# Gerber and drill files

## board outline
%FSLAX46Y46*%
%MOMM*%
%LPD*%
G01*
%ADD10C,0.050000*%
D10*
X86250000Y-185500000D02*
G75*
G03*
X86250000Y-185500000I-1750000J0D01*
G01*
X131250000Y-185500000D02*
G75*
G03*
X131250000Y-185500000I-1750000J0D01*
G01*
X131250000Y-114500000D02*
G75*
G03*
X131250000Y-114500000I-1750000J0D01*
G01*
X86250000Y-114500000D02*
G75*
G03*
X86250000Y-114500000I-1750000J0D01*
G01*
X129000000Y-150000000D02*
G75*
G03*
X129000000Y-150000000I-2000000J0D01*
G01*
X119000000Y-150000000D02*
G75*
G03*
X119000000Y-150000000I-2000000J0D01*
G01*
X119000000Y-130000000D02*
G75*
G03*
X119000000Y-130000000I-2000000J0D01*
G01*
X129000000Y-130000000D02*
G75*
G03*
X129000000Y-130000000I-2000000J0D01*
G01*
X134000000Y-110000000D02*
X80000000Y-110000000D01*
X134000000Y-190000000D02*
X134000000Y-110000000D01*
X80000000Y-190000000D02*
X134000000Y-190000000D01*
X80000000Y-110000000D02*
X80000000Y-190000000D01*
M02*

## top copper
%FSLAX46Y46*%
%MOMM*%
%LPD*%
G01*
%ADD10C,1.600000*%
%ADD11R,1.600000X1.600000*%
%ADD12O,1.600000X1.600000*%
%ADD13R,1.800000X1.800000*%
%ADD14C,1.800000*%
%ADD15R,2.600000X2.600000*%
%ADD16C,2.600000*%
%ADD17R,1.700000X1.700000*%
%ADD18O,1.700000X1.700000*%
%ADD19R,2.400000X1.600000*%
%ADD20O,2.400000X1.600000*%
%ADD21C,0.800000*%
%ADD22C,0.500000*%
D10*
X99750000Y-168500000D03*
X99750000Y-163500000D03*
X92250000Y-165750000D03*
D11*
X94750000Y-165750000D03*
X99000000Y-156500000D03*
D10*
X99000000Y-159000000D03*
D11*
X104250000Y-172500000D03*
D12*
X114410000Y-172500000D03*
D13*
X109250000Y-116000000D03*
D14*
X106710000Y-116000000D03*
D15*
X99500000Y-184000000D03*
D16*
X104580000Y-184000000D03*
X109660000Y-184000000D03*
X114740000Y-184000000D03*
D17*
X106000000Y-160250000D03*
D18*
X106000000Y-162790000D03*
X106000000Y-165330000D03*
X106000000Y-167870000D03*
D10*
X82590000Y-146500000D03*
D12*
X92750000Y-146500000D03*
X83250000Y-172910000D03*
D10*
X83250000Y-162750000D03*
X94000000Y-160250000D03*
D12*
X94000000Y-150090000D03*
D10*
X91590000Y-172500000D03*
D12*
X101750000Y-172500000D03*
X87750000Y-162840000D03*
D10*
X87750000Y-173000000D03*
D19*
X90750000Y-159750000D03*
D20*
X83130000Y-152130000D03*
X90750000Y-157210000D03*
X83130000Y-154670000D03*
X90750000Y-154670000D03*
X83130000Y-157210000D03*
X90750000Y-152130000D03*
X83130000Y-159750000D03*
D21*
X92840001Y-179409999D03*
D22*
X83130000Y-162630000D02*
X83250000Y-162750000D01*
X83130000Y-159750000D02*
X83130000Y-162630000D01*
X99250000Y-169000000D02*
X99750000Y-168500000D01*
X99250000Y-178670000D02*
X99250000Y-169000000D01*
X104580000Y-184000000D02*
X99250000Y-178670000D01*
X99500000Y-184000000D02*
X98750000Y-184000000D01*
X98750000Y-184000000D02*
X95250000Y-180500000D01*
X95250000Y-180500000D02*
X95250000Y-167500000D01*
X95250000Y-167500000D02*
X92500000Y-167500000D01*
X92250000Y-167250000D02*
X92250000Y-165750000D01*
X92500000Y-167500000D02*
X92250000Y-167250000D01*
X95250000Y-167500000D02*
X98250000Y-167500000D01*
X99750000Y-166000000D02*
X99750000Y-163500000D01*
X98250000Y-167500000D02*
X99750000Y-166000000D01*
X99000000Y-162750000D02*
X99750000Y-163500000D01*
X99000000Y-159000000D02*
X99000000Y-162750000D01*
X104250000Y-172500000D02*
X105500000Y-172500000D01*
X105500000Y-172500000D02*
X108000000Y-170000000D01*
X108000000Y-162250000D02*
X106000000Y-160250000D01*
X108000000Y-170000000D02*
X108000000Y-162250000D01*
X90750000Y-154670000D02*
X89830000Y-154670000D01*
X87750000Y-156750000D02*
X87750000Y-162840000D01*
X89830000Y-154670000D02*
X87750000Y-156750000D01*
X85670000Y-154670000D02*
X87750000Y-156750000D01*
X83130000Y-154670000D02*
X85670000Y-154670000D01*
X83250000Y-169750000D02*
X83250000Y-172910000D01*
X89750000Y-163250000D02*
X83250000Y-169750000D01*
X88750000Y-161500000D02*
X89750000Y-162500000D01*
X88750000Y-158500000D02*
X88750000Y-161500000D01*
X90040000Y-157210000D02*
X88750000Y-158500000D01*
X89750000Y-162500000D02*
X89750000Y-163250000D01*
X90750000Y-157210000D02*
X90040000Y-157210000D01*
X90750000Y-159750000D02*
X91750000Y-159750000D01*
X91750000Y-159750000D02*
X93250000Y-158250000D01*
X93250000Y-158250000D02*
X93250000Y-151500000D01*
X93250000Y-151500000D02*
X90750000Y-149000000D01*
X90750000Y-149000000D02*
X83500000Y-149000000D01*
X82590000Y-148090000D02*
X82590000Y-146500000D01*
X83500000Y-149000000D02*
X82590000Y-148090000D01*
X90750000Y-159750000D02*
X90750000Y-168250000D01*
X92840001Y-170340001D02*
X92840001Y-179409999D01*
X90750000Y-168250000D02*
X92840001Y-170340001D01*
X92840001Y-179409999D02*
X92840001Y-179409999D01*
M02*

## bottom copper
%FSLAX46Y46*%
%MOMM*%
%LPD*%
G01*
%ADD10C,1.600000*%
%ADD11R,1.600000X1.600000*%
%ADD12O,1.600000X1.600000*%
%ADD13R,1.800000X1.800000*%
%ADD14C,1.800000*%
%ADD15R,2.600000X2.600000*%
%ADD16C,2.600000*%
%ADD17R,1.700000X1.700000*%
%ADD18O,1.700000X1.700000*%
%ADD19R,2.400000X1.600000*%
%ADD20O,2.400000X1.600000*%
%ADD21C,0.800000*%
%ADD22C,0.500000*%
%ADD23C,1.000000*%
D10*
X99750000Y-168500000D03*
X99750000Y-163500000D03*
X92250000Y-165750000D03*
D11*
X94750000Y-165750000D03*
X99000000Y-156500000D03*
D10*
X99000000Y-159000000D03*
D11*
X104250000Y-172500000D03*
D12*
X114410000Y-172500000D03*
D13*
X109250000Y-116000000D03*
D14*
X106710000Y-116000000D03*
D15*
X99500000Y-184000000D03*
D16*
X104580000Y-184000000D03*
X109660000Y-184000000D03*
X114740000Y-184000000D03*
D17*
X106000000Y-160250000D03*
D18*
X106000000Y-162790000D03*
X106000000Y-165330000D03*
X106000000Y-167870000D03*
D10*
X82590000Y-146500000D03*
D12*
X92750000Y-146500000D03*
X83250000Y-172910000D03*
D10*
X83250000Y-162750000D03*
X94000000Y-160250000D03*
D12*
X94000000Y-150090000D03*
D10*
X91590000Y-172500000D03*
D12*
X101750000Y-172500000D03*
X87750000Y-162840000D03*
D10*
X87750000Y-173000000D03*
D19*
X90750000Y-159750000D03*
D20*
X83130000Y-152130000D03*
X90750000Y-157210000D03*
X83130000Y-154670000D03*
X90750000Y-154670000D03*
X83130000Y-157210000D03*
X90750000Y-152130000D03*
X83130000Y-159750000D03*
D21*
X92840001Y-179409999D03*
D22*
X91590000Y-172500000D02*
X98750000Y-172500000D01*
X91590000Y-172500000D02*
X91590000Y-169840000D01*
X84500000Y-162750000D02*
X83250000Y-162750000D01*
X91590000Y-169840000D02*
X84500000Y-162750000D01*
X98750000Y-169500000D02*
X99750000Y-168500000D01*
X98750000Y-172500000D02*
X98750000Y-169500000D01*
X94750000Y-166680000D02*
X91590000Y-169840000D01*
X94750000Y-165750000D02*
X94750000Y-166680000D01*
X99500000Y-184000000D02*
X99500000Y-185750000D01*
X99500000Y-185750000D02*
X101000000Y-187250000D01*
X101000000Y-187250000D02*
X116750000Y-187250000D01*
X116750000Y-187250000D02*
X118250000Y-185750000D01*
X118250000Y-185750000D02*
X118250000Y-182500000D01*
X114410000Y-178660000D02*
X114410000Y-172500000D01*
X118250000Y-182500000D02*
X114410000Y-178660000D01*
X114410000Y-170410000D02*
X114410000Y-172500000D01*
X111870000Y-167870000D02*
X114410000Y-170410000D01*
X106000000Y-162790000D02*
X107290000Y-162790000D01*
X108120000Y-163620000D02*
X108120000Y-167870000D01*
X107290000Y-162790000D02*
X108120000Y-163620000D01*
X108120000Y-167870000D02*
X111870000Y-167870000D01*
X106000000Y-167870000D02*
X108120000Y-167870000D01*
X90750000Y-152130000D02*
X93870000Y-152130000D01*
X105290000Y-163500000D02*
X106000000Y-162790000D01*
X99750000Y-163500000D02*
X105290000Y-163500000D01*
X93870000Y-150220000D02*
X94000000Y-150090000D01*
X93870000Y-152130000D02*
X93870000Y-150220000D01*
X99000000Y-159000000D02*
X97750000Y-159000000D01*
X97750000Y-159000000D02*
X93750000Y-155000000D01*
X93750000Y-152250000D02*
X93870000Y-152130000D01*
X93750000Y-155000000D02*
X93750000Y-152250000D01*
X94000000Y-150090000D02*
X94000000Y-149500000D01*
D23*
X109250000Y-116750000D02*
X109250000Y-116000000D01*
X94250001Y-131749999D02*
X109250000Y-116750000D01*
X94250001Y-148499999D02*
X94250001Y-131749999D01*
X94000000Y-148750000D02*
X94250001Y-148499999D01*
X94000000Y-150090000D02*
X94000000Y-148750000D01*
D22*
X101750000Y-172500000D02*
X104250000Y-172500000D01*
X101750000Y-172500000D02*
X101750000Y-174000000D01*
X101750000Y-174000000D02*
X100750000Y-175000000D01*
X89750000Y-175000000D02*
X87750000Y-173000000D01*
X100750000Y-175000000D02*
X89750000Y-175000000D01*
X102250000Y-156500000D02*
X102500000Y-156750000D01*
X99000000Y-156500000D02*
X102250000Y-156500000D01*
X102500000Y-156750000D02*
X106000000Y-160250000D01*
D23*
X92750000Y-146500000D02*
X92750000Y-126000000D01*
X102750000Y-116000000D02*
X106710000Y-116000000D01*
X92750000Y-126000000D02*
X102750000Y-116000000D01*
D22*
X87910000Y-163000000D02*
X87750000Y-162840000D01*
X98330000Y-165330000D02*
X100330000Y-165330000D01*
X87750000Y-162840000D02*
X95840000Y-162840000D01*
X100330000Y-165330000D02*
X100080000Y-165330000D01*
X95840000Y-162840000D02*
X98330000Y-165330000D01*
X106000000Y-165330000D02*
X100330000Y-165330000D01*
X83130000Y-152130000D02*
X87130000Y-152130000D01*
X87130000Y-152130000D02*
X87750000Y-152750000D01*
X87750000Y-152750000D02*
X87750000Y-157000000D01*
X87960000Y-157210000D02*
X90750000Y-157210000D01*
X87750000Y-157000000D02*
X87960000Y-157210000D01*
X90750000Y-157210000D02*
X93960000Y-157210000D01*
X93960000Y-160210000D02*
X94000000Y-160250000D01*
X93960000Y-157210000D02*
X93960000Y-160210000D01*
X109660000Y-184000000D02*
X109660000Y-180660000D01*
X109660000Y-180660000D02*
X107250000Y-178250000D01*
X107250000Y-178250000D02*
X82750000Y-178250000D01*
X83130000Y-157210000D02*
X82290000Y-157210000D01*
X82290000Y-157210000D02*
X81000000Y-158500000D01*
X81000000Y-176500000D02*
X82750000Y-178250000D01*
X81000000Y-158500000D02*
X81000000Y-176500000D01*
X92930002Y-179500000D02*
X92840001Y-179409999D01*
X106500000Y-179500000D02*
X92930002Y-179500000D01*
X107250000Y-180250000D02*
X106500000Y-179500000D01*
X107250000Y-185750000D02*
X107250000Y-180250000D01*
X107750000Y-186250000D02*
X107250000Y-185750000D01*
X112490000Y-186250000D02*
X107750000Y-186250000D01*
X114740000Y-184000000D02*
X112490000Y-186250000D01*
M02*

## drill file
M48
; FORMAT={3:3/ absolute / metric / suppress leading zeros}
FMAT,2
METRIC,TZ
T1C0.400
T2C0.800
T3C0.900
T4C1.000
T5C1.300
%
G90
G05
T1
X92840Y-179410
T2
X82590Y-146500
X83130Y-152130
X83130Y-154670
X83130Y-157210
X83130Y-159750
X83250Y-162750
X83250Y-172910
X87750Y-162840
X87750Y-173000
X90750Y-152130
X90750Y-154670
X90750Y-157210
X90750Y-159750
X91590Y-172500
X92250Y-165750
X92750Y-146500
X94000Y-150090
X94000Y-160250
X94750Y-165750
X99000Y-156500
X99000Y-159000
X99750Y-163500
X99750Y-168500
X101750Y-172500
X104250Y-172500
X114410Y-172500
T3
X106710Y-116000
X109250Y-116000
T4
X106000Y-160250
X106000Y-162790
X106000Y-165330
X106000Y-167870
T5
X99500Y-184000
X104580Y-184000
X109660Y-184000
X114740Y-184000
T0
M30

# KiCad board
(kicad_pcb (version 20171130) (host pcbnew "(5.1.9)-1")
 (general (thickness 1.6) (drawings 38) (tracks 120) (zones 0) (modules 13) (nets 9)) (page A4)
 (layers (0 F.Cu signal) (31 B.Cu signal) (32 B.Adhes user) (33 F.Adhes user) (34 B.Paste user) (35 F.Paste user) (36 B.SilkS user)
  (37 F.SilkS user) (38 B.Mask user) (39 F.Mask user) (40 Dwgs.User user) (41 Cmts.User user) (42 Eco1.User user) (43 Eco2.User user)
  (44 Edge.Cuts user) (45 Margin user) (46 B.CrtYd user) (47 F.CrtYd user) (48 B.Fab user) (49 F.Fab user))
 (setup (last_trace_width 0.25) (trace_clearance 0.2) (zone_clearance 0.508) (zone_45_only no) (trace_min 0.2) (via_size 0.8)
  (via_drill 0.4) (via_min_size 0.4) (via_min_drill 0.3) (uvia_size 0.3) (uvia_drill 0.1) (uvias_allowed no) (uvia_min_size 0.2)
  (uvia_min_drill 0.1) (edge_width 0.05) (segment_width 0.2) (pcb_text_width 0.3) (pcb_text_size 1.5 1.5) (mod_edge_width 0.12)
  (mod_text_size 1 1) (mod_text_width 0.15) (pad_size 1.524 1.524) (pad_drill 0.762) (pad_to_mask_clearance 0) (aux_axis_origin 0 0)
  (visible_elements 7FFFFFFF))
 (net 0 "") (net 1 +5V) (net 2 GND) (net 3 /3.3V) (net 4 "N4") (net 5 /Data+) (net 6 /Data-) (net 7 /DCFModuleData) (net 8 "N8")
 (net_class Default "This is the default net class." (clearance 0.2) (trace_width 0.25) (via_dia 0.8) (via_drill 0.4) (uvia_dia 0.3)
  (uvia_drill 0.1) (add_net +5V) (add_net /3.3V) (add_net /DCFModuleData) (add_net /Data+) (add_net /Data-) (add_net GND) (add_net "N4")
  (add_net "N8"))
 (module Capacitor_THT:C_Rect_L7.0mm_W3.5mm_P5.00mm (layer F.Cu) (at 99.75 168.5 90)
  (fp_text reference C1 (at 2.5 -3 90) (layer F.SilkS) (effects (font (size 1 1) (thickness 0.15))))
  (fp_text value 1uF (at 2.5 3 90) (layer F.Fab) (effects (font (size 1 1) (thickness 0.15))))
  (pad 1 thru_hole circle (at 0 0 90) (size 1.6 1.6) (drill 0.8) (layers *.Cu *.Mask) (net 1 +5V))
  (pad 2 thru_hole circle (at 5 0 90) (size 1.6 1.6) (drill 0.8) (layers *.Cu *.Mask) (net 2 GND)))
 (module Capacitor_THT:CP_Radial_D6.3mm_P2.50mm (layer F.Cu) (at 94.75 165.75 180)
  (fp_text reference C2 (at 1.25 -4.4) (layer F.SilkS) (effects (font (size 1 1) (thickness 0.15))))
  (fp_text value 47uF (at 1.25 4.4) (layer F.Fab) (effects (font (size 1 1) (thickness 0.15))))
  (pad 2 thru_hole circle (at 2.5 0 180) (size 1.6 1.6) (drill 0.8) (layers *.Cu *.Mask) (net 2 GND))
  (pad 1 thru_hole rect (at 0 0 180) (size 1.6 1.6) (drill 0.8) (layers *.Cu *.Mask) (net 1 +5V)))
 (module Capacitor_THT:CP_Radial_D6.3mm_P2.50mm (layer F.Cu) (at 99 156.5 270)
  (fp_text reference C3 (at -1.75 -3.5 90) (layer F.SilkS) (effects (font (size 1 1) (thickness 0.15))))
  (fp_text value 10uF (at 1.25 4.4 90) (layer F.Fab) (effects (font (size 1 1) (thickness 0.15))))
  (pad 1 thru_hole rect (at 0 0 270) (size 1.6 1.6) (drill 0.8) (layers *.Cu *.Mask) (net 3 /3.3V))
  (pad 2 thru_hole circle (at 2.5 0 270) (size 1.6 1.6) (drill 0.8) (layers *.Cu *.Mask) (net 2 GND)))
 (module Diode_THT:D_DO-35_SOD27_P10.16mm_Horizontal (layer F.Cu) (at 104.25 172.5)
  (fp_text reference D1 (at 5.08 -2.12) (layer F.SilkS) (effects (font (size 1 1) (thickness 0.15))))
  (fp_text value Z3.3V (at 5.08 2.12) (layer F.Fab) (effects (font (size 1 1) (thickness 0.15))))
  (pad 1 thru_hole rect (at 0 0) (size 1.6 1.6) (drill 0.8) (layers *.Cu *.Mask) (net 3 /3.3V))
  (pad 2 thru_hole oval (at 10.16 0) (size 1.6 1.6) (drill 0.8) (layers *.Cu *.Mask) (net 2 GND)))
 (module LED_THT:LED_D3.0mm (layer F.Cu) (at 109.25 116 180)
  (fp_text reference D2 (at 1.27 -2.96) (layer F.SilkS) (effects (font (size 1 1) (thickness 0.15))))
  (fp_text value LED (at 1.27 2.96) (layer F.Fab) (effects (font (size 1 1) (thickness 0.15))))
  (pad 1 thru_hole rect (at 0 0 180) (size 1.8 1.8) (drill 0.9) (layers *.Cu *.Mask) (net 2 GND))
  (pad 2 thru_hole circle (at 2.54 0 180) (size 1.8 1.8) (drill 0.9) (layers *.Cu *.Mask) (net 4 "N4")))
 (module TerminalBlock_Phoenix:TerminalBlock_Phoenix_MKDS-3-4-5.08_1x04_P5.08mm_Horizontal (layer F.Cu) (at 99.5 184)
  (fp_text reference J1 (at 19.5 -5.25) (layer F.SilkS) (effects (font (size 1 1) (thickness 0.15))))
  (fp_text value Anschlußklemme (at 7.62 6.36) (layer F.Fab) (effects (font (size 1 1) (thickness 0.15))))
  (pad 1 thru_hole rect (at 0 0) (size 2.6 2.6) (drill 1.3) (layers *.Cu *.Mask) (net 2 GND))
  (pad 2 thru_hole circle (at 5.08 0) (size 2.6 2.6) (drill 1.3) (layers *.Cu *.Mask) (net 1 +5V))
  (pad 3 thru_hole circle (at 10.16 0) (size 2.6 2.6) (drill 1.3) (layers *.Cu *.Mask) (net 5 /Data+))
  (pad 4 thru_hole circle (at 15.24 0) (size 2.6 2.6) (drill 1.3) (layers *.Cu *.Mask) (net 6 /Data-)))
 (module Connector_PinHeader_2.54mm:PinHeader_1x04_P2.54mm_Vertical (layer F.Cu) (at 106 160.25)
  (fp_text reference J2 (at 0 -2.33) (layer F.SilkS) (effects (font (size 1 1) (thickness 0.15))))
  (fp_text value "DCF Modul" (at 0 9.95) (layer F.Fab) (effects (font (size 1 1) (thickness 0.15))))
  (pad 1 thru_hole rect (at 0 0) (size 1.7 1.7) (drill 1) (layers *.Cu *.Mask) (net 3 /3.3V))
  (pad 2 thru_hole oval (at 0 2.54) (size 1.7 1.7) (drill 1) (layers *.Cu *.Mask) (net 2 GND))
  (pad 3 thru_hole oval (at 0 5.08) (size 1.7 1.7) (drill 1) (layers *.Cu *.Mask) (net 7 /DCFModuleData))
  (pad 4 thru_hole oval (at 0 7.62) (size 1.7 1.7) (drill 1) (layers *.Cu *.Mask) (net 2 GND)))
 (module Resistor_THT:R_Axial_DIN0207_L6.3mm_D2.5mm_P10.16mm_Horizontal (layer F.Cu) (at 82.59 146.5)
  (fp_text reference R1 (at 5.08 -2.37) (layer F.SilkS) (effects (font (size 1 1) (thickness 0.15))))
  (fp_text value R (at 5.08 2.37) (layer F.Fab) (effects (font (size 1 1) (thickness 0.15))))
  (pad 1 thru_hole circle (at 0 0) (size 1.6 1.6) (drill 0.8) (layers *.Cu *.Mask) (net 6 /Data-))
  (pad 2 thru_hole oval (at 10.16 0) (size 1.6 1.6) (drill 0.8) (layers *.Cu *.Mask) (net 4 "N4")))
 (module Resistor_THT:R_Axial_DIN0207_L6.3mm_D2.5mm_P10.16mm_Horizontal (layer F.Cu) (at 83.25 162.75 270)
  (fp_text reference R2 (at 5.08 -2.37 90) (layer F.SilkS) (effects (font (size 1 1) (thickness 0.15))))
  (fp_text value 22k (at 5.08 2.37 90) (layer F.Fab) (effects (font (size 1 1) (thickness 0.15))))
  (pad 2 thru_hole oval (at 10.16 0 270) (size 1.6 1.6) (drill 0.8) (layers *.Cu *.Mask) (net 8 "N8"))
  (pad 1 thru_hole circle (at 0 0 270) (size 1.6 1.6) (drill 0.8) (layers *.Cu *.Mask) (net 1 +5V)))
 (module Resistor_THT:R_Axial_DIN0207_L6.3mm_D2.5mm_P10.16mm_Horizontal (layer F.Cu) (at 94 160.25 90)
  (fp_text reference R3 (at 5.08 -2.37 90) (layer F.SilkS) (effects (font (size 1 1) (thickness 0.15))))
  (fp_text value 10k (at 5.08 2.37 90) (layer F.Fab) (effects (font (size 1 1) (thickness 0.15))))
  (pad 1 thru_hole circle (at 0 0 90) (size 1.6 1.6) (drill 0.8) (layers *.Cu *.Mask) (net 8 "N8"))
  (pad 2 thru_hole oval (at 10.16 0 90) (size 1.6 1.6) (drill 0.8) (layers *.Cu *.Mask) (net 2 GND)))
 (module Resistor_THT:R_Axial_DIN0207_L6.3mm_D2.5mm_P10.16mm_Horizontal (layer F.Cu) (at 91.59 172.5)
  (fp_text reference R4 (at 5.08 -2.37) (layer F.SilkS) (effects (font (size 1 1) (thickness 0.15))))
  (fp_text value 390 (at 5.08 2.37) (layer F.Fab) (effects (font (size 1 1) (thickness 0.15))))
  (pad 1 thru_hole circle (at 0 0) (size 1.6 1.6) (drill 0.8) (layers *.Cu *.Mask) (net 1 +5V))
  (pad 2 thru_hole oval (at 10.16 0) (size 1.6 1.6) (drill 0.8) (layers *.Cu *.Mask) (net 3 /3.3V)))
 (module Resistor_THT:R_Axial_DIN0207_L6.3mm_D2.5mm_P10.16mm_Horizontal (layer F.Cu) (at 87.75 173 90)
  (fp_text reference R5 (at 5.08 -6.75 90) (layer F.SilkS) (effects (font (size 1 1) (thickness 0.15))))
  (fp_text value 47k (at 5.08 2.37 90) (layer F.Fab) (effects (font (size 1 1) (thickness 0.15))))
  (pad 2 thru_hole oval (at 10.16 0 90) (size 1.6 1.6) (drill 0.8) (layers *.Cu *.Mask) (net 7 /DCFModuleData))
  (pad 1 thru_hole circle (at 0 0 90) (size 1.6 1.6) (drill 0.8) (layers *.Cu *.Mask) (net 3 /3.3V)))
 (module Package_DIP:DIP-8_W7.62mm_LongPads (layer F.Cu) (at 90.75 159.75 180)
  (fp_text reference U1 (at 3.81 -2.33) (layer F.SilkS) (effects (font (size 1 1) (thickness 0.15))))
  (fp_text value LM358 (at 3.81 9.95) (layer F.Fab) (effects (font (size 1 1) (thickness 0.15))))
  (pad 1 thru_hole rect (at 0 0 180) (size 2.4 1.6) (drill 0.8) (layers *.Cu *.Mask) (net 6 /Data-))
  (pad 5 thru_hole oval (at 7.62 7.62 180) (size 2.4 1.6) (drill 0.8) (layers *.Cu *.Mask) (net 8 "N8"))
  (pad 2 thru_hole oval (at 0 2.54 180) (size 2.4 1.6) (drill 0.8) (layers *.Cu *.Mask) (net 8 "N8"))
  (pad 6 thru_hole oval (at 7.62 5.08 180) (size 2.4 1.6) (drill 0.8) (layers *.Cu *.Mask) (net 7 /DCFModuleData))
  (pad 3 thru_hole oval (at 0 5.08 180) (size 2.4 1.6) (drill 0.8) (layers *.Cu *.Mask) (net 7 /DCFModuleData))
  (pad 7 thru_hole oval (at 7.62 2.54 180) (size 2.4 1.6) (drill 0.8) (layers *.Cu *.Mask) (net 5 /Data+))
  (pad 4 thru_hole oval (at 0 7.62 180) (size 2.4 1.6) (drill 0.8) (layers *.Cu *.Mask) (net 2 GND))
  (pad 8 thru_hole oval (at 7.62 0 180) (size 2.4 1.6) (drill 0.8) (layers *.Cu *.Mask) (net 1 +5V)))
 (gr_circle (center 84.5 185.5) (end 86.25 185.5) (layer Edge.Cuts) (width 0.05))
 (gr_circle (center 129.5 185.5) (end 131.25 185.5) (layer Edge.Cuts) (width 0.05))
 (gr_circle (center 129.5 114.5) (end 131.25 114.5) (layer Edge.Cuts) (width 0.05))
 (gr_circle (center 84.5 114.5) (end 86.25 114.5) (layer Edge.Cuts) (width 0.05))
 (gr_circle (center 127 150) (end 129 150) (layer Edge.Cuts) (width 0.05))
 (gr_circle (center 117 150) (end 119 150) (layer Edge.Cuts) (width 0.05))
 (gr_circle (center 117 130) (end 119 130) (layer Edge.Cuts) (width 0.05))
 (gr_circle (center 127 130) (end 129 130) (layer Edge.Cuts) (width 0.05))
 (gr_line (start 134 110) (end 80 110) (layer Edge.Cuts) (width 0.05))
 (gr_line (start 134 190) (end 134 110) (layer Edge.Cuts) (width 0.05))
 (gr_line (start 80 190) (end 134 190) (layer Edge.Cuts) (width 0.05))
 (gr_line (start 80 110) (end 80 190) (layer Edge.Cuts) (width 0.05))
 (segment (start 91.59 172.5) (end 98.75 172.5) (width 0.5) (layer B.Cu) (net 1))
 (segment (start 83.13 162.63) (end 83.25 162.75) (width 0.5) (layer F.Cu) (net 1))
 (segment (start 83.13 159.75) (end 83.13 162.63) (width 0.5) (layer F.Cu) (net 1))
 (segment (start 91.59 172.5) (end 91.59 169.84) (width 0.5) (layer B.Cu) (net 1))
 (segment (start 84.5 162.75) (end 83.25 162.75) (width 0.5) (layer B.Cu) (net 1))
 (segment (start 91.59 169.84) (end 84.5 162.75) (width 0.5) (layer B.Cu) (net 1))
 (segment (start 98.75 169.5) (end 99.75 168.5) (width 0.5) (layer B.Cu) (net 1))
 (segment (start 98.75 172.5) (end 98.75 169.5) (width 0.5) (layer B.Cu) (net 1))
 (segment (start 99.25 169) (end 99.75 168.5) (width 0.5) (layer F.Cu) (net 1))
 (segment (start 99.25 178.67) (end 99.25 169) (width 0.5) (layer F.Cu) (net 1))
 (segment (start 104.58 184) (end 99.25 178.67) (width 0.5) (layer F.Cu) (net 1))
 (segment (start 94.75 166.68) (end 91.59 169.84) (width 0.5) (layer B.Cu) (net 1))
 (segment (start 94.75 165.75) (end 94.75 166.68) (width 0.5) (layer B.Cu) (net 1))
 (segment (start 99.5 184) (end 99.5 185.75) (width 0.5) (layer B.Cu) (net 2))
 (segment (start 99.5 185.75) (end 101 187.25) (width 0.5) (layer B.Cu) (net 2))
 (segment (start 101 187.25) (end 116.75 187.25) (width 0.5) (layer B.Cu) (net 2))
 (segment (start 116.75 187.25) (end 118.25 185.75) (width 0.5) (layer B.Cu) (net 2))
 (segment (start 118.25 185.75) (end 118.25 182.5) (width 0.5) (layer B.Cu) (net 2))
 (segment (start 114.41 178.66) (end 114.41 172.5) (width 0.5) (layer B.Cu) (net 2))
 (segment (start 118.25 182.5) (end 114.41 178.66) (width 0.5) (layer B.Cu) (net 2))
 (segment (start 114.41 170.41) (end 114.41 172.5) (width 0.5) (layer B.Cu) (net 2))
 (segment (start 111.87 167.87) (end 114.41 170.41) (width 0.5) (layer B.Cu) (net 2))
 (segment (start 106 162.79) (end 107.29 162.79) (width 0.5) (layer B.Cu) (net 2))
 (segment (start 108.12 163.62) (end 108.12 167.87) (width 0.5) (layer B.Cu) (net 2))
 (segment (start 107.29 162.79) (end 108.12 163.62) (width 0.5) (layer B.Cu) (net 2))
 (segment (start 108.12 167.87) (end 111.87 167.87) (width 0.5) (layer B.Cu) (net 2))
 (segment (start 106 167.87) (end 108.12 167.87) (width 0.5) (layer B.Cu) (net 2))
 (segment (start 99.5 184) (end 98.75 184) (width 0.5) (layer F.Cu) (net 2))
 (segment (start 98.75 184) (end 95.25 180.5) (width 0.5) (layer F.Cu) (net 2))
 (segment (start 95.25 180.5) (end 95.25 167.5) (width 0.5) (layer F.Cu) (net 2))
 (segment (start 90.75 152.13) (end 93.87 152.13) (width 0.5) (layer B.Cu) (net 2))
 (segment (start 105.29 163.5) (end 106 162.79) (width 0.5) (layer B.Cu) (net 2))
 (segment (start 99.75 163.5) (end 105.29 163.5) (width 0.5) (layer B.Cu) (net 2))
 (segment (start 95.25 167.5) (end 92.5 167.5) (width 0.5) (layer F.Cu) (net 2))
 (segment (start 92.25 167.25) (end 92.25 165.75) (width 0.5) (layer F.Cu) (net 2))
 (segment (start 92.5 167.5) (end 92.25 167.25) (width 0.5) (layer F.Cu) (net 2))
 (segment (start 95.25 167.5) (end 98.25 167.5) (width 0.5) (layer F.Cu) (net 2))
 (segment (start 99.75 166) (end 99.75 163.5) (width 0.5) (layer F.Cu) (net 2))
 (segment (start 98.25 167.5) (end 99.75 166) (width 0.5) (layer F.Cu) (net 2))
 (segment (start 93.87 150.22) (end 94 150.09) (width 0.5) (layer B.Cu) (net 2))
 (segment (start 93.87 152.13) (end 93.87 150.22) (width 0.5) (layer B.Cu) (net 2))
 (segment (start 99 159) (end 97.75 159) (width 0.5) (layer B.Cu) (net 2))
 (segment (start 97.75 159) (end 93.75 155) (width 0.5) (layer B.Cu) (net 2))
 (segment (start 93.75 152.25) (end 93.87 152.13) (width 0.5) (layer B.Cu) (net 2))
 (segment (start 93.75 155) (end 93.75 152.25) (width 0.5) (layer B.Cu) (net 2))
 (segment (start 99 162.75) (end 99.75 163.5) (width 0.5) (layer F.Cu) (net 2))
 (segment (start 99 159) (end 99 162.75) (width 0.5) (layer F.Cu) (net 2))
 (segment (start 94 150.09) (end 94 149.5) (width 0.5) (layer B.Cu) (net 2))
 (segment (start 109.25 116.75) (end 109.25 116) (width 1) (layer B.Cu) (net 2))
 (segment (start 94.250001 131.749999) (end 109.25 116.75) (width 1) (layer B.Cu) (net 2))
 (segment (start 94.250001 148.499999) (end 94.250001 131.749999) (width 1) (layer B.Cu) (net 2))
 (segment (start 94 148.75) (end 94.250001 148.499999) (width 1) (layer B.Cu) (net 2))
 (segment (start 94 150.09) (end 94 148.75) (width 1) (layer B.Cu) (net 2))
 (segment (start 104.25 172.5) (end 105.5 172.5) (width 0.5) (layer F.Cu) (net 3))
 (segment (start 105.5 172.5) (end 108 170) (width 0.5) (layer F.Cu) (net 3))
 (segment (start 108 162.25) (end 106 160.25) (width 0.5) (layer F.Cu) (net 3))
 (segment (start 108 170) (end 108 162.25) (width 0.5) (layer F.Cu) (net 3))
 (segment (start 101.75 172.5) (end 104.25 172.5) (width 0.5) (layer B.Cu) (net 3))
 (segment (start 101.75 172.5) (end 101.75 174) (width 0.5) (layer B.Cu) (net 3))
 (segment (start 101.75 174) (end 100.75 175) (width 0.5) (layer B.Cu) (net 3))
 (segment (start 89.75 175) (end 87.75 173) (width 0.5) (layer B.Cu) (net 3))
 (segment (start 100.75 175) (end 89.75 175) (width 0.5) (layer B.Cu) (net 3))
 (segment (start 102.25 156.5) (end 102.5 156.75) (width 0.5) (layer B.Cu) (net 3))
 (segment (start 99 156.5) (end 102.25 156.5) (width 0.5) (layer B.Cu) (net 3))
 (segment (start 102.5 156.75) (end 106 160.25) (width 0.5) (layer B.Cu) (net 3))
 (segment (start 92.75 146.5) (end 92.75 126) (width 1) (layer B.Cu) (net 4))
 (segment (start 102.75 116) (end 106.71 116) (width 1) (layer B.Cu) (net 4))
 (segment (start 92.75 126) (end 102.75 116) (width 1) (layer B.Cu) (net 4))
 (segment (start 90.75 154.67) (end 89.83 154.67) (width 0.5) (layer F.Cu) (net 7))
 (segment (start 87.75 156.75) (end 87.75 162.84) (width 0.5) (layer F.Cu) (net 7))
 (segment (start 89.83 154.67) (end 87.75 156.75) (width 0.5) (layer F.Cu) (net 7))
 (segment (start 85.67 154.67) (end 87.75 156.75) (width 0.5) (layer F.Cu) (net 7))
 (segment (start 83.13 154.67) (end 85.67 154.67) (width 0.5) (layer F.Cu) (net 7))
 (segment (start 87.91 163) (end 87.75 162.84) (width 0.5) (layer B.Cu) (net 7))
 (segment (start 98.33 165.33) (end 100.33 165.33) (width 0.5) (layer B.Cu) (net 7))
 (segment (start 87.75 162.84) (end 95.84 162.84) (width 0.5) (layer B.Cu) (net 7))
 (segment (start 100.33 165.33) (end 100.08 165.33) (width 0.5) (layer B.Cu) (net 7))
 (segment (start 95.84 162.84) (end 98.33 165.33) (width 0.5) (layer B.Cu) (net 7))
 (segment (start 106 165.33) (end 100.33 165.33) (width 0.5) (layer B.Cu) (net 7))
 (segment (start 83.13 152.13) (end 87.13 152.13) (width 0.5) (layer B.Cu) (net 8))
 (segment (start 87.13 152.13) (end 87.75 152.75) (width 0.5) (layer B.Cu) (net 8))
 (segment (start 87.75 152.75) (end 87.75 157) (width 0.5) (layer B.Cu) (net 8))
 (segment (start 87.96 157.21) (end 90.75 157.21) (width 0.5) (layer B.Cu) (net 8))
 (segment (start 87.75 157) (end 87.96 157.21) (width 0.5) (layer B.Cu) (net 8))
 (segment (start 90.75 157.21) (end 93.96 157.21) (width 0.5) (layer B.Cu) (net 8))
 (segment (start 83.25 169.75) (end 83.25 172.91) (width 0.5) (layer F.Cu) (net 8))
 (segment (start 89.75 163.25) (end 83.25 169.75) (width 0.5) (layer F.Cu) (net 8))
 (segment (start 88.75 161.5) (end 89.75 162.5) (width 0.5) (layer F.Cu) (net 8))
 (segment (start 88.75 158.5) (end 88.75 161.5) (width 0.5) (layer F.Cu) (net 8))
 (segment (start 90.04 157.21) (end 88.75 158.5) (width 0.5) (layer F.Cu) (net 8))
 (segment (start 89.75 162.5) (end 89.75 163.25) (width 0.5) (layer F.Cu) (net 8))
 (segment (start 90.75 157.21) (end 90.04 157.21) (width 0.5) (layer F.Cu) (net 8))
 (segment (start 93.96 160.21) (end 94 160.25) (width 0.5) (layer B.Cu) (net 8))
 (segment (start 93.96 157.21) (end 93.96 160.21) (width 0.5) (layer B.Cu) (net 8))
 (segment (start 109.66 184) (end 109.66 180.66) (width 0.5) (layer B.Cu) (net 5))
 (segment (start 109.66 180.66) (end 107.25 178.25) (width 0.5) (layer B.Cu) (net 5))
 (segment (start 107.25 178.25) (end 82.75 178.25) (width 0.5) (layer B.Cu) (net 5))
 (segment (start 83.13 157.21) (end 82.29 157.21) (width 0.5) (layer B.Cu) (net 5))
 (segment (start 82.29 157.21) (end 81 158.5) (width 0.5) (layer B.Cu) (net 5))
 (segment (start 81 176.5) (end 82.75 178.25) (width 0.5) (layer B.Cu) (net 5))
 (segment (start 81 158.5) (end 81 176.5) (width 0.5) (layer B.Cu) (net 5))
 (segment (start 90.75 159.75) (end 91.75 159.75) (width 0.5) (layer F.Cu) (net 6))
 (segment (start 91.75 159.75) (end 93.25 158.25) (width 0.5) (layer F.Cu) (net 6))
 (segment (start 93.25 158.25) (end 93.25 151.5) (width 0.5) (layer F.Cu) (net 6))
 (segment (start 93.25 151.5) (end 90.75 149) (width 0.5) (layer F.Cu) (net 6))
 (segment (start 90.75 149) (end 83.5 149) (width 0.5) (layer F.Cu) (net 6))
 (segment (start 82.59 148.09) (end 82.59 146.5) (width 0.5) (layer F.Cu) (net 6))
 (segment (start 83.5 149) (end 82.59 148.09) (width 0.5) (layer F.Cu) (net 6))
 (segment (start 90.75 159.75) (end 90.75 168.25) (width 0.5) (layer F.Cu) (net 6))
 (segment (start 92.840001 170.340001) (end 92.840001 179.409999) (width 0.5) (layer F.Cu) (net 6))
 (segment (start 90.75 168.25) (end 92.840001 170.340001) (width 0.5) (layer F.Cu) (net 6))
 (segment (start 92.840001 179.409999) (end 92.840001 179.409999) (width 0.5) (layer F.Cu) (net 6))
 (via (at 92.840001 179.409999) (size 0.8) (drill 0.4) (layers F.Cu B.Cu) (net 6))
 (segment (start 92.930002 179.5) (end 92.840001 179.409999) (width 0.5) (layer B.Cu) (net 6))
 (segment (start 106.5 179.5) (end 92.930002 179.5) (width 0.5) (layer B.Cu) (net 6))
 (segment (start 107.25 180.25) (end 106.5 179.5) (width 0.5) (layer B.Cu) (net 6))
 (segment (start 107.25 185.75) (end 107.25 180.25) (width 0.5) (layer B.Cu) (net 6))
 (segment (start 107.75 186.25) (end 107.25 185.75) (width 0.5) (layer B.Cu) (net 6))
 (segment (start 112.49 186.25) (end 107.75 186.25) (width 0.5) (layer B.Cu) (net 6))
 (segment (start 114.74 184) (end 112.49 186.25) (width 0.5) (layer B.Cu) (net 6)))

